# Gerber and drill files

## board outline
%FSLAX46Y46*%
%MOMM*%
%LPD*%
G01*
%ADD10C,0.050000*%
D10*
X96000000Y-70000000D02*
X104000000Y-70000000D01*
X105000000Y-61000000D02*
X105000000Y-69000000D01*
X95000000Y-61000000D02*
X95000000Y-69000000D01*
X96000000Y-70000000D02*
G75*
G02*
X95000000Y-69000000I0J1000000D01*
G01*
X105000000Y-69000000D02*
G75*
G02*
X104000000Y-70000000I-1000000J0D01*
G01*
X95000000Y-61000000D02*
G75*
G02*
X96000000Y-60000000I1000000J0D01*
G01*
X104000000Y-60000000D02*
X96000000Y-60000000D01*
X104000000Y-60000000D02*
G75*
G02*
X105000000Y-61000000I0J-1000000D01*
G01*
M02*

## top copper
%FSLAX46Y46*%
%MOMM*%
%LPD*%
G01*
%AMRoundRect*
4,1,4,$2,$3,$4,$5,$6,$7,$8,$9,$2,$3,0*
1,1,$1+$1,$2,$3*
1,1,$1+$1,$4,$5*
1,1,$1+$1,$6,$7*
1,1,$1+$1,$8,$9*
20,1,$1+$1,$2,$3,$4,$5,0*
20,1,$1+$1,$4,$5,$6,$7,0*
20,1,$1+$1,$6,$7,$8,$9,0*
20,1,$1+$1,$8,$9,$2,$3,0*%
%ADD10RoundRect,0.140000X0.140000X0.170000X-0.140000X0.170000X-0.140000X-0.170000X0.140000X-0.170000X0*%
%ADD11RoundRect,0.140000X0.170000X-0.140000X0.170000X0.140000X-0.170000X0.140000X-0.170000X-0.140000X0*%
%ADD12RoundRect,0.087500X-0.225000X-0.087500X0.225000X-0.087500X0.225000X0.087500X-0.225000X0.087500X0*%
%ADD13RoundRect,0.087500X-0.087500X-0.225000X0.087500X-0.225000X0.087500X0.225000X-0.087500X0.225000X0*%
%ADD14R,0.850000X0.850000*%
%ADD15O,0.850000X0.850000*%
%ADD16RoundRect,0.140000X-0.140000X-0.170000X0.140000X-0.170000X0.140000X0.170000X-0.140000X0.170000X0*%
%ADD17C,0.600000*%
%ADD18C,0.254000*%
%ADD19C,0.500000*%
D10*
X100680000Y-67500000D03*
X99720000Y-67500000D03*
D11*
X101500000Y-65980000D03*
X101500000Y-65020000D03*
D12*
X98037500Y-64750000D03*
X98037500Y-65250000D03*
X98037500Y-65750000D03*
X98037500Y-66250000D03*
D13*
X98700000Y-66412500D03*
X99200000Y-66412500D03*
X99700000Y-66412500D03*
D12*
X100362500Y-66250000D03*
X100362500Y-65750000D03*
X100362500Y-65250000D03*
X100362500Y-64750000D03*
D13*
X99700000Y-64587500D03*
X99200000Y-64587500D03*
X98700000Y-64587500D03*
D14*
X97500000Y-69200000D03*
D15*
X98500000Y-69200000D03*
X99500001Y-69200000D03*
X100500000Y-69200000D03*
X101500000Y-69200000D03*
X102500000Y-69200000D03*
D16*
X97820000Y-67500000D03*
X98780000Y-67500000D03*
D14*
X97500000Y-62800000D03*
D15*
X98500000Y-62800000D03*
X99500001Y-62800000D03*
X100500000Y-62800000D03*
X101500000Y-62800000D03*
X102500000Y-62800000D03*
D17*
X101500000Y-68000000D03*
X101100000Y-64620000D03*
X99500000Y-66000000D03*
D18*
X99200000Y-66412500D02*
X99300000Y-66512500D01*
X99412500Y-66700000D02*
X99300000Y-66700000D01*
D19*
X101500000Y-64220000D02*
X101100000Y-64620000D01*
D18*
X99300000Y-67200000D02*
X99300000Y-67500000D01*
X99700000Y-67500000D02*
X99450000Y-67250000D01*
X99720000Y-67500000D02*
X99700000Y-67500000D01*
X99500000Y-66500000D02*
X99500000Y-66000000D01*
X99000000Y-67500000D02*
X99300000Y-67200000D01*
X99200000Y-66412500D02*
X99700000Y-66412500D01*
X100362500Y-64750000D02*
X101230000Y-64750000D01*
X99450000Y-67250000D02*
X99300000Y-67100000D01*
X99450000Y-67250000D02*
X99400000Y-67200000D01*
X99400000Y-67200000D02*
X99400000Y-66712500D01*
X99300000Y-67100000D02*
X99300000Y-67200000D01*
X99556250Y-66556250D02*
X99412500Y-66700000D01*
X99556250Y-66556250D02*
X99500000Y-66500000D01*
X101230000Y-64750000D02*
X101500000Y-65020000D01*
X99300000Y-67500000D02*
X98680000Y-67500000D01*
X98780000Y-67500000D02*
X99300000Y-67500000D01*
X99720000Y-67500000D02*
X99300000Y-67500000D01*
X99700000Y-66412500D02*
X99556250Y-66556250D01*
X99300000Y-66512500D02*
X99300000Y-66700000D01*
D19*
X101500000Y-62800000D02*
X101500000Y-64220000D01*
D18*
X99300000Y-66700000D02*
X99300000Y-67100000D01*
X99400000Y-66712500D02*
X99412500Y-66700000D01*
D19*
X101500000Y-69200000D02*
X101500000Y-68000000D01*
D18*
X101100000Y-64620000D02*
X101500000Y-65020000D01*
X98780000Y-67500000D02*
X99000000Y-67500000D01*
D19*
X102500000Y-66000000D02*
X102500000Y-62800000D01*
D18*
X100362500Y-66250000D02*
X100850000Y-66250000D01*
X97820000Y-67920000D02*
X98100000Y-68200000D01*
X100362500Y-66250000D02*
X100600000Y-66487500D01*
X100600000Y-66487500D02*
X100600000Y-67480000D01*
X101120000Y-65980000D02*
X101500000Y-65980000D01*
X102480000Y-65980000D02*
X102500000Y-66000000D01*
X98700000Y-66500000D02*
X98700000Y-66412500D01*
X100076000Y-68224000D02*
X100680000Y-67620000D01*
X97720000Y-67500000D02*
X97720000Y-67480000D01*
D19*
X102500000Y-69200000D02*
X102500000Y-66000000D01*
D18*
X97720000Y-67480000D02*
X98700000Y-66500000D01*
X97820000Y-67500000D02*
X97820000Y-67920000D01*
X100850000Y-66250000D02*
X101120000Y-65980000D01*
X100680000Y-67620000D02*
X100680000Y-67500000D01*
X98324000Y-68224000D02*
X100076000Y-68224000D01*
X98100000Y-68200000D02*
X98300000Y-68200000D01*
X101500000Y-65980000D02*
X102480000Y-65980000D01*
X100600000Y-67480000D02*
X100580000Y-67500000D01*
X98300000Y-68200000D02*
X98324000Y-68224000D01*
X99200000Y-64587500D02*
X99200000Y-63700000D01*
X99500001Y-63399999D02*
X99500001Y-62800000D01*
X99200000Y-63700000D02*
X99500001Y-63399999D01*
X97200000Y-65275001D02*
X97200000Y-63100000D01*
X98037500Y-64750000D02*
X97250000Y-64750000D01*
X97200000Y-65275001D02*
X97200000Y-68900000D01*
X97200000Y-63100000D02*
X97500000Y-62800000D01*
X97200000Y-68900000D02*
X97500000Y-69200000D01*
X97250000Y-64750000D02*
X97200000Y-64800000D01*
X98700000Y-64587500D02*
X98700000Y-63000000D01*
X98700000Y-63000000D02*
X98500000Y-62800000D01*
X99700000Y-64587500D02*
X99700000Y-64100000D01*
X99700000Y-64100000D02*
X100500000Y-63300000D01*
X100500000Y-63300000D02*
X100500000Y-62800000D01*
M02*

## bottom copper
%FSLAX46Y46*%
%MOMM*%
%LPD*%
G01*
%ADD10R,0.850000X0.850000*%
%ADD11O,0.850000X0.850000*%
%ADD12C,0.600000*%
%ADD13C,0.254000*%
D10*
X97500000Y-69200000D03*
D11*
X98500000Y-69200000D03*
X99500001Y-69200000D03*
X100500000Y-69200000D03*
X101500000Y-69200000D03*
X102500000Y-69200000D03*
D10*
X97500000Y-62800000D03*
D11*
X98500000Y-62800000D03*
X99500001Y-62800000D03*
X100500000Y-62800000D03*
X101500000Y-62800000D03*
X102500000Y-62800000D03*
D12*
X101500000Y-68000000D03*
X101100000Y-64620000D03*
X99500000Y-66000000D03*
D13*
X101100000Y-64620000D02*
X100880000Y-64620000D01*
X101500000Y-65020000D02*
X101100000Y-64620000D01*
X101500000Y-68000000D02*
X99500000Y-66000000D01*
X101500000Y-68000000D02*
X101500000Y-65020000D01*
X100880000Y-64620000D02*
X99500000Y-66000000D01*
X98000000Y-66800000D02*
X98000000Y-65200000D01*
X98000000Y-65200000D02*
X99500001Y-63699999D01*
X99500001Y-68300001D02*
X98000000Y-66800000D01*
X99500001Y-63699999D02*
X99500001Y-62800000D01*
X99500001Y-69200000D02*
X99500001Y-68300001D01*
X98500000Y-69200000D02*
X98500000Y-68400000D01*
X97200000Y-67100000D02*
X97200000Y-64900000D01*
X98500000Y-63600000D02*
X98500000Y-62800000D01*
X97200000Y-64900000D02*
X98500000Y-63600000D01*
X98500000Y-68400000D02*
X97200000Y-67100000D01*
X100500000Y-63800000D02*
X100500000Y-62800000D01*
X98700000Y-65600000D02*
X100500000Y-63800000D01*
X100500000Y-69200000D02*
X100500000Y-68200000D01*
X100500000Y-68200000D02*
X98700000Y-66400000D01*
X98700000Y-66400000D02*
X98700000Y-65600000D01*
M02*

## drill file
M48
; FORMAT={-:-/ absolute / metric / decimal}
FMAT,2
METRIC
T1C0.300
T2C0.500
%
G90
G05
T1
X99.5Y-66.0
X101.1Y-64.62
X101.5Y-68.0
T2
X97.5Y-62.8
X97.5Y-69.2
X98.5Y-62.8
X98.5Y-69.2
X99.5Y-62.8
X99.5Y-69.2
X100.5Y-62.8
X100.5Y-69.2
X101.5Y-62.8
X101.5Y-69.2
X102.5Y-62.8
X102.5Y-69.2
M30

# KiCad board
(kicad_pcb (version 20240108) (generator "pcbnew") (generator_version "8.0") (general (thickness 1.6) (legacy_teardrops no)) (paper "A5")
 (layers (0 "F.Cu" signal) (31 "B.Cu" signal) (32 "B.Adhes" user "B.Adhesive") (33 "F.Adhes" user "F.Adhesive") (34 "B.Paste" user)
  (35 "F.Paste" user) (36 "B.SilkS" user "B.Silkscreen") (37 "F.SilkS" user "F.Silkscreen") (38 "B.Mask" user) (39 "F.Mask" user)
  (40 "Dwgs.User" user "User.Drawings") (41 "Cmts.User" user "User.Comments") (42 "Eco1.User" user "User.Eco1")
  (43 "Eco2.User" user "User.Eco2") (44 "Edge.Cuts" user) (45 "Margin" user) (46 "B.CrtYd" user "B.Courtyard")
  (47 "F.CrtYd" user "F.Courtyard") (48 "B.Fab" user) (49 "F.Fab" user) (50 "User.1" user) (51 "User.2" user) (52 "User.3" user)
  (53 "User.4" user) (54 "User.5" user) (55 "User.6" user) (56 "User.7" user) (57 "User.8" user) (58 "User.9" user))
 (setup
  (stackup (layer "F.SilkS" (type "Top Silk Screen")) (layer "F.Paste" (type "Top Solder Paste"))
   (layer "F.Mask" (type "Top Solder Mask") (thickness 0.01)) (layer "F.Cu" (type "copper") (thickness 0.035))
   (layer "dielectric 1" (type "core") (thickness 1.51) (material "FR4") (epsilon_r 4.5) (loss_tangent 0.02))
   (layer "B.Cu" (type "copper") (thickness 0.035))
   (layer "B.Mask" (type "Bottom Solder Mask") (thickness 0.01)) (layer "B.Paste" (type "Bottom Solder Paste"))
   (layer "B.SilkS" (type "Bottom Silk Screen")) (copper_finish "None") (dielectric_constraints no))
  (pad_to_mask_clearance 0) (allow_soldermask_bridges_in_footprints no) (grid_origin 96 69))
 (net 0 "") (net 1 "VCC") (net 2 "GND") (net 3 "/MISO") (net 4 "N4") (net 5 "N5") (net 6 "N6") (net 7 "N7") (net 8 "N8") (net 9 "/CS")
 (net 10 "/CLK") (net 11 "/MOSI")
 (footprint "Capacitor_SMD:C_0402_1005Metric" (layer "F.Cu") (at 100.2 67.5 180)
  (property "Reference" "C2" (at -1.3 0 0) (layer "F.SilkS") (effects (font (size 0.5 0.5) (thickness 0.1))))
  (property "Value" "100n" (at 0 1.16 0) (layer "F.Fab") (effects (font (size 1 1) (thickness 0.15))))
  (pad "1" smd roundrect (at -0.48 0 180) (size 0.56 0.62) (layers "F.Cu" "F.Paste" "F.Mask") (roundrect_rratio 0.25) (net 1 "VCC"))
  (pad "2" smd roundrect (at 0.48 0 180) (size 0.56 0.62) (layers "F.Cu" "F.Paste" "F.Mask") (roundrect_rratio 0.25) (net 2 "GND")))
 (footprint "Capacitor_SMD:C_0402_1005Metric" (layer "F.Cu") (at 101.5 65.5 90)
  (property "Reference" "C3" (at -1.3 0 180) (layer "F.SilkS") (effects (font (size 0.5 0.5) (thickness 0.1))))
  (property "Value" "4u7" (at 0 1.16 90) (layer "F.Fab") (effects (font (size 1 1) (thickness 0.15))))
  (pad "1" smd roundrect (at -0.48 0 90) (size 0.56 0.62) (layers "F.Cu" "F.Paste" "F.Mask") (roundrect_rratio 0.25) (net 1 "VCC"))
  (pad "2" smd roundrect (at 0.48 0 90) (size 0.56 0.62) (layers "F.Cu" "F.Paste" "F.Mask") (roundrect_rratio 0.25) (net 2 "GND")))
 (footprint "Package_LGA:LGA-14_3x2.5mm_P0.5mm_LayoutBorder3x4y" (layer "F.Cu") (at 99.2 65.5)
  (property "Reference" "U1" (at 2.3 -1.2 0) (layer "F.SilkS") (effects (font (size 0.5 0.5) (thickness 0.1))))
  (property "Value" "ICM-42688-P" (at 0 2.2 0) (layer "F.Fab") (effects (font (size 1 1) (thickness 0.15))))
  (pad "1" smd roundrect (at -1.1625 -0.75) (size 0.625 0.35) (layers "F.Cu" "F.Paste" "F.Mask") (roundrect_rratio 0.25) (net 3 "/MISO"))
  (pad "2" smd roundrect (at -1.1625 -0.25) (size 0.625 0.35) (layers "F.Cu" "F.Paste" "F.Mask") (roundrect_rratio 0.25) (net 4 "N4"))
  (pad "3" smd roundrect (at -1.1625 0.25) (size 0.625 0.35) (layers "F.Cu" "F.Paste" "F.Mask") (roundrect_rratio 0.25) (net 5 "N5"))
  (pad "4" smd roundrect (at -1.1625 0.75) (size 0.625 0.35) (layers "F.Cu" "F.Paste" "F.Mask") (roundrect_rratio 0.25) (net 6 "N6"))
  (pad "5" smd roundrect (at -0.5 0.9125) (size 0.35 0.625) (layers "F.Cu" "F.Paste" "F.Mask") (roundrect_rratio 0.25) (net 1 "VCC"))
  (pad "6" smd roundrect (at 0 0.9125) (size 0.35 0.625) (layers "F.Cu" "F.Paste" "F.Mask") (roundrect_rratio 0.25) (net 2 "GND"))
  (pad "7" smd roundrect (at 0.5 0.9125) (size 0.35 0.625) (layers "F.Cu" "F.Paste" "F.Mask") (roundrect_rratio 0.25) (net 2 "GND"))
  (pad "8" smd roundrect (at 1.1625 0.75) (size 0.625 0.35) (layers "F.Cu" "F.Paste" "F.Mask") (roundrect_rratio 0.25) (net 1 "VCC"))
  (pad "9" smd roundrect (at 1.1625 0.25) (size 0.625 0.35) (layers "F.Cu" "F.Paste" "F.Mask") (roundrect_rratio 0.25) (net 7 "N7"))
  (pad "10" smd roundrect (at 1.1625 -0.25) (size 0.625 0.35) (layers "F.Cu" "F.Paste" "F.Mask") (roundrect_rratio 0.25) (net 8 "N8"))
  (pad "11" smd roundrect (at 1.1625 -0.75) (size 0.625 0.35) (layers "F.Cu" "F.Paste" "F.Mask") (roundrect_rratio 0.25) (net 2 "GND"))
  (pad "12" smd roundrect (at 0.5 -0.9125) (size 0.35 0.625) (layers "F.Cu" "F.Paste" "F.Mask") (roundrect_rratio 0.25) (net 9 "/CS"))
  (pad "13" smd roundrect (at 0 -0.9125) (size 0.35 0.625) (layers "F.Cu" "F.Paste" "F.Mask") (roundrect_rratio 0.25) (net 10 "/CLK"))
  (pad "14" smd roundrect (at -0.5 -0.9125) (size 0.35 0.625) (layers "F.Cu" "F.Paste" "F.Mask") (roundrect_rratio 0.25) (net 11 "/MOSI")))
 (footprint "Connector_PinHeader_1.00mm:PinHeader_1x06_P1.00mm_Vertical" (layer "F.Cu") (at 97.5 69.2 90)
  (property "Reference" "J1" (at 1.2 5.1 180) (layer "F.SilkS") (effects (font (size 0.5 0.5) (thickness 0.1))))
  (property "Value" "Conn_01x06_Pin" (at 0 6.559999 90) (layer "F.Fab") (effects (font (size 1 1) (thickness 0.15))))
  (pad "1" thru_hole rect (at 0 0 90) (size 0.85 0.85) (drill 0.5) (layers "*.Cu" "*.Mask") (remove_unused_layers no) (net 3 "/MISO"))
  (pad "2" thru_hole oval (at 0 1 90) (size 0.85 0.85) (drill 0.5) (layers "*.Cu" "*.Mask") (remove_unused_layers no) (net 11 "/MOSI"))
  (pad "3" thru_hole oval (at 0 2.000001 90) (size 0.85 0.85) (drill 0.5) (layers "*.Cu" "*.Mask") (remove_unused_layers no) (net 10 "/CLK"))
  (pad "4" thru_hole oval (at 0 3 90) (size 0.85 0.85) (drill 0.5) (layers "*.Cu" "*.Mask") (remove_unused_layers no) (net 9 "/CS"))
  (pad "5" thru_hole oval (at 0 4 90) (size 0.85 0.85) (drill 0.5) (layers "*.Cu" "*.Mask") (remove_unused_layers no) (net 2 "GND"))
  (pad "6" thru_hole oval (at 0 5 90) (size 0.85 0.85) (drill 0.5) (layers "*.Cu" "*.Mask") (remove_unused_layers no) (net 1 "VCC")))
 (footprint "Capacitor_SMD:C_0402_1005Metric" (layer "F.Cu") (at 98.3 67.5)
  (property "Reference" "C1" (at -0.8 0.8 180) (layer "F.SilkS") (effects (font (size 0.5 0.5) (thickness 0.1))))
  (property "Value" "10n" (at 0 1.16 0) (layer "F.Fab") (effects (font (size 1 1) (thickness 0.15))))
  (pad "1" smd roundrect (at -0.48 0) (size 0.56 0.62) (layers "F.Cu" "F.Paste" "F.Mask") (roundrect_rratio 0.25) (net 1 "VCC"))
  (pad "2" smd roundrect (at 0.48 0) (size 0.56 0.62) (layers "F.Cu" "F.Paste" "F.Mask") (roundrect_rratio 0.25) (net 2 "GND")))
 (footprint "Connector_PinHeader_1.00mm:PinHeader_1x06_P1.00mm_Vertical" (layer "F.Cu") (at 97.5 62.8 90)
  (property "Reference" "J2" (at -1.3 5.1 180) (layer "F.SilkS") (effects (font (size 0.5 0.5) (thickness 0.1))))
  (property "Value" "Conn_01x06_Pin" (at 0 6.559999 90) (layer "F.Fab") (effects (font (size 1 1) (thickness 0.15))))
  (pad "1" thru_hole rect (at 0 0 90) (size 0.85 0.85) (drill 0.5) (layers "*.Cu" "*.Mask") (remove_unused_layers no) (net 3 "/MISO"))
  (pad "2" thru_hole oval (at 0 1 90) (size 0.85 0.85) (drill 0.5) (layers "*.Cu" "*.Mask") (remove_unused_layers no) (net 11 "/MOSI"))
  (pad "3" thru_hole oval (at 0 2.000001 90) (size 0.85 0.85) (drill 0.5) (layers "*.Cu" "*.Mask") (remove_unused_layers no) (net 10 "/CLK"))
  (pad "4" thru_hole oval (at 0 3 90) (size 0.85 0.85) (drill 0.5) (layers "*.Cu" "*.Mask") (remove_unused_layers no) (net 9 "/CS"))
  (pad "5" thru_hole oval (at 0 4 90) (size 0.85 0.85) (drill 0.5) (layers "*.Cu" "*.Mask") (remove_unused_layers no) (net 2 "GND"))
  (pad "6" thru_hole oval (at 0 5 90) (size 0.85 0.85) (drill 0.5) (layers "*.Cu" "*.Mask") (remove_unused_layers no) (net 1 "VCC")))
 (gr_line (start 96 70) (end 104 70) (stroke (width 0.05) (type default)) (layer "Edge.Cuts"))
 (gr_line (start 105 61) (end 105 69) (stroke (width 0.05) (type default)) (layer "Edge.Cuts"))
 (gr_line (start 95 61) (end 95 69) (stroke (width 0.05) (type default)) (layer "Edge.Cuts"))
 (gr_arc (start 96 70) (mid 95.292893 69.707107) (end 95 69) (stroke (width 0.05) (type default)) (layer "Edge.Cuts"))
 (gr_arc (start 105 69) (mid 104.707107 69.707107) (end 104 70) (stroke (width 0.05) (type default)) (layer "Edge.Cuts"))
 (gr_arc (start 95 61) (mid 95.292893 60.292893) (end 96 60) (stroke (width 0.05) (type default)) (layer "Edge.Cuts"))
 (gr_line (start 104 60) (end 96 60) (stroke (width 0.05) (type default)) (layer "Edge.Cuts"))
 (gr_arc (start 104 60) (mid 104.707107 60.292893) (end 105 61) (stroke (width 0.05) (type default)) (layer "Edge.Cuts"))
 (segment (start 99.2 66.4125) (end 99.3 66.5125) (width 0.254) (layer "F.Cu") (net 2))
 (segment (start 99.4125 66.7) (end 99.3 66.7) (width 0.254) (layer "F.Cu") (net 2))
 (segment (start 101.5 64.22) (end 101.1 64.62) (width 0.5) (layer "F.Cu") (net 2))
 (segment (start 99.3 67.2) (end 99.3 67.5) (width 0.254) (layer "F.Cu") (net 2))
 (segment (start 99.7 67.5) (end 99.45 67.25) (width 0.254) (layer "F.Cu") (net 2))
 (segment (start 99.72 67.5) (end 99.7 67.5) (width 0.254) (layer "F.Cu") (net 2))
 (segment (start 99.5 66.5) (end 99.5 66) (width 0.254) (layer "F.Cu") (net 2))
 (segment (start 99 67.5) (end 99.3 67.2) (width 0.254) (layer "F.Cu") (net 2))
 (segment (start 99.2 66.4125) (end 99.7 66.4125) (width 0.254) (layer "F.Cu") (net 2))
 (segment (start 100.3625 64.75) (end 101.23 64.75) (width 0.254) (layer "F.Cu") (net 2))
 (segment (start 99.45 67.25) (end 99.3 67.1) (width 0.254) (layer "F.Cu") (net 2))
 (segment (start 99.45 67.25) (end 99.4 67.2) (width 0.254) (layer "F.Cu") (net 2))
 (segment (start 99.4 67.2) (end 99.4 66.7125) (width 0.254) (layer "F.Cu") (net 2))
 (segment (start 99.3 67.1) (end 99.3 67.2) (width 0.254) (layer "F.Cu") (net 2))
 (segment (start 99.55625 66.55625) (end 99.4125 66.7) (width 0.254) (layer "F.Cu") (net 2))
 (segment (start 99.55625 66.55625) (end 99.5 66.5) (width 0.254) (layer "F.Cu") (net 2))
 (segment (start 101.23 64.75) (end 101.5 65.02) (width 0.254) (layer "F.Cu") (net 2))
 (segment (start 99.3 67.5) (end 98.68 67.5) (width 0.254) (layer "F.Cu") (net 2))
 (segment (start 98.78 67.5) (end 99.3 67.5) (width 0.254) (layer "F.Cu") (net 2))
 (segment (start 99.72 67.5) (end 99.3 67.5) (width 0.254) (layer "F.Cu") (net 2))
 (segment (start 99.7 66.4125) (end 99.55625 66.55625) (width 0.254) (layer "F.Cu") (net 2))
 (segment (start 99.3 66.5125) (end 99.3 66.7) (width 0.254) (layer "F.Cu") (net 2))
 (segment (start 101.5 62.8) (end 101.5 64.22) (width 0.5) (layer "F.Cu") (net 2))
 (segment (start 99.3 66.7) (end 99.3 67.1) (width 0.254) (layer "F.Cu") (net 2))
 (segment (start 99.4 66.7125) (end 99.4125 66.7) (width 0.254) (layer "F.Cu") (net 2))
 (segment (start 101.5 69.2) (end 101.5 68) (width 0.5) (layer "F.Cu") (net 2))
 (segment (start 101.1 64.62) (end 101.5 65.02) (width 0.254) (layer "F.Cu") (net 2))
 (segment (start 98.78 67.5) (end 99 67.5) (width 0.254) (layer "F.Cu") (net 2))
 (via (at 101.5 68) (size 0.6) (drill 0.3) (layers "F.Cu" "B.Cu") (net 2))
 (via (at 101.1 64.62) (size 0.6) (drill 0.3) (layers "F.Cu" "B.Cu") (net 2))
 (via (at 99.5 66) (size 0.6) (drill 0.3) (layers "F.Cu" "B.Cu") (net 2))
 (segment (start 101.1 64.62) (end 100.88 64.62) (width 0.254) (layer "B.Cu") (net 2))
 (segment (start 101.5 65.02) (end 101.1 64.62) (width 0.254) (layer "B.Cu") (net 2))
 (segment (start 101.5 68) (end 99.5 66) (width 0.254) (layer "B.Cu") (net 2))
 (segment (start 101.5 68) (end 101.5 65.02) (width 0.254) (layer "B.Cu") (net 2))
 (segment (start 100.88 64.62) (end 99.5 66) (width 0.254) (layer "B.Cu") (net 2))
 (segment (start 102.5 66) (end 102.5 62.8) (width 0.5) (layer "F.Cu") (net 1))
 (segment (start 100.3625 66.25) (end 100.85 66.25) (width 0.254) (layer "F.Cu") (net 1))
 (segment (start 97.82 67.92) (end 98.1 68.2) (width 0.254) (layer "F.Cu") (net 1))
 (segment (start 100.3625 66.25) (end 100.6 66.4875) (width 0.254) (layer "F.Cu") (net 1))
 (segment (start 100.6 66.4875) (end 100.6 67.48) (width 0.254) (layer "F.Cu") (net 1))
 (segment (start 101.12 65.98) (end 101.5 65.98) (width 0.254) (layer "F.Cu") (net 1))
 (segment (start 102.48 65.98) (end 102.5 66) (width 0.254) (layer "F.Cu") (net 1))
 (segment (start 98.7 66.5) (end 98.7 66.4125) (width 0.254) (layer "F.Cu") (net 1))
 (segment (start 100.076 68.224) (end 100.68 67.62) (width 0.254) (layer "F.Cu") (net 1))
 (segment (start 97.72 67.5) (end 97.72 67.48) (width 0.254) (layer "F.Cu") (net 1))
 (segment (start 102.5 69.2) (end 102.5 66) (width 0.5) (layer "F.Cu") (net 1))
 (segment (start 97.72 67.48) (end 98.7 66.5) (width 0.254) (layer "F.Cu") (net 1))
 (segment (start 97.82 67.5) (end 97.82 67.92) (width 0.254) (layer "F.Cu") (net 1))
 (segment (start 100.85 66.25) (end 101.12 65.98) (width 0.254) (layer "F.Cu") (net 1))
 (segment (start 100.68 67.62) (end 100.68 67.5) (width 0.254) (layer "F.Cu") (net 1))
 (segment (start 98.324 68.224) (end 100.076 68.224) (width 0.254) (layer "F.Cu") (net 1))
 (segment (start 98.1 68.2) (end 98.3 68.2) (width 0.254) (layer "F.Cu") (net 1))
 (segment (start 101.5 65.98) (end 102.48 65.98) (width 0.254) (layer "F.Cu") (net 1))
 (segment (start 100.6 67.48) (end 100.58 67.5) (width 0.254) (layer "F.Cu") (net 1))
 (segment (start 98.3 68.2) (end 98.324 68.224) (width 0.254) (layer "F.Cu") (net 1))
 (segment (start 99.2 64.5875) (end 99.2 63.7) (width 0.254) (layer "F.Cu") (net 10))
 (segment (start 99.500001 63.399999) (end 99.500001 62.8) (width 0.254) (layer "F.Cu") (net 10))
 (segment (start 99.2 63.7) (end 99.500001 63.399999) (width 0.254) (layer "F.Cu") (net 10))
 (segment (start 98 66.8) (end 98 65.2) (width 0.254) (layer "B.Cu") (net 10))
 (segment (start 98 65.2) (end 99.500001 63.699999) (width 0.254) (layer "B.Cu") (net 10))
 (segment (start 99.500001 68.300001) (end 98 66.8) (width 0.254) (layer "B.Cu") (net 10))
 (segment (start 99.500001 63.699999) (end 99.500001 62.8) (width 0.254) (layer "B.Cu") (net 10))
 (segment (start 99.500001 69.2) (end 99.500001 68.300001) (width 0.254) (layer "B.Cu") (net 10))
 (segment (start 97.2 65.275001) (end 97.2 63.1) (width 0.254) (layer "F.Cu") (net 3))
 (segment (start 98.0375 64.75) (end 97.25 64.75) (width 0.254) (layer "F.Cu") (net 3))
 (segment (start 97.2 65.275001) (end 97.2 68.9) (width 0.254) (layer "F.Cu") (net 3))
 (segment (start 97.2 63.1) (end 97.5 62.8) (width 0.254) (layer "F.Cu") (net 3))
 (segment (start 97.2 68.9) (end 97.5 69.2) (width 0.254) (layer "F.Cu") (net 3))
 (segment (start 97.25 64.75) (end 97.2 64.8) (width 0.254) (layer "F.Cu") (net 3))
 (segment (start 98.7 64.5875) (end 98.7 63) (width 0.254) (layer "F.Cu") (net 11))
 (segment (start 98.7 63) (end 98.5 62.8) (width 0.254) (layer "F.Cu") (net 11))
 (segment (start 98.5 69.2) (end 98.5 68.4) (width 0.254) (layer "B.Cu") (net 11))
 (segment (start 97.2 67.1) (end 97.2 64.9) (width 0.254) (layer "B.Cu") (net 11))
 (segment (start 98.5 63.6) (end 98.5 62.8) (width 0.254) (layer "B.Cu") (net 11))
 (segment (start 97.2 64.9) (end 98.5 63.6) (width 0.254) (layer "B.Cu") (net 11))
 (segment (start 98.5 68.4) (end 97.2 67.1) (width 0.254) (layer "B.Cu") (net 11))
 (segment (start 99.7 64.5875) (end 99.7 64.1) (width 0.254) (layer "F.Cu") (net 9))
 (segment (start 99.7 64.1) (end 100.5 63.3) (width 0.254) (layer "F.Cu") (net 9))
 (segment (start 100.5 63.3) (end 100.5 62.8) (width 0.254) (layer "F.Cu") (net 9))
 (segment (start 100.5 63.8) (end 100.5 62.8) (width 0.254) (layer "B.Cu") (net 9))
 (segment (start 98.7 65.6) (end 100.5 63.8) (width 0.254) (layer "B.Cu") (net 9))
 (segment (start 100.5 69.2) (end 100.5 68.2) (width 0.254) (layer "B.Cu") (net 9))
 (segment (start 100.5 68.2) (end 98.7 66.4) (width 0.254) (layer "B.Cu") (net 9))
 (segment (start 98.7 66.4) (end 98.7 65.6) (width 0.254) (layer "B.Cu") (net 9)))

